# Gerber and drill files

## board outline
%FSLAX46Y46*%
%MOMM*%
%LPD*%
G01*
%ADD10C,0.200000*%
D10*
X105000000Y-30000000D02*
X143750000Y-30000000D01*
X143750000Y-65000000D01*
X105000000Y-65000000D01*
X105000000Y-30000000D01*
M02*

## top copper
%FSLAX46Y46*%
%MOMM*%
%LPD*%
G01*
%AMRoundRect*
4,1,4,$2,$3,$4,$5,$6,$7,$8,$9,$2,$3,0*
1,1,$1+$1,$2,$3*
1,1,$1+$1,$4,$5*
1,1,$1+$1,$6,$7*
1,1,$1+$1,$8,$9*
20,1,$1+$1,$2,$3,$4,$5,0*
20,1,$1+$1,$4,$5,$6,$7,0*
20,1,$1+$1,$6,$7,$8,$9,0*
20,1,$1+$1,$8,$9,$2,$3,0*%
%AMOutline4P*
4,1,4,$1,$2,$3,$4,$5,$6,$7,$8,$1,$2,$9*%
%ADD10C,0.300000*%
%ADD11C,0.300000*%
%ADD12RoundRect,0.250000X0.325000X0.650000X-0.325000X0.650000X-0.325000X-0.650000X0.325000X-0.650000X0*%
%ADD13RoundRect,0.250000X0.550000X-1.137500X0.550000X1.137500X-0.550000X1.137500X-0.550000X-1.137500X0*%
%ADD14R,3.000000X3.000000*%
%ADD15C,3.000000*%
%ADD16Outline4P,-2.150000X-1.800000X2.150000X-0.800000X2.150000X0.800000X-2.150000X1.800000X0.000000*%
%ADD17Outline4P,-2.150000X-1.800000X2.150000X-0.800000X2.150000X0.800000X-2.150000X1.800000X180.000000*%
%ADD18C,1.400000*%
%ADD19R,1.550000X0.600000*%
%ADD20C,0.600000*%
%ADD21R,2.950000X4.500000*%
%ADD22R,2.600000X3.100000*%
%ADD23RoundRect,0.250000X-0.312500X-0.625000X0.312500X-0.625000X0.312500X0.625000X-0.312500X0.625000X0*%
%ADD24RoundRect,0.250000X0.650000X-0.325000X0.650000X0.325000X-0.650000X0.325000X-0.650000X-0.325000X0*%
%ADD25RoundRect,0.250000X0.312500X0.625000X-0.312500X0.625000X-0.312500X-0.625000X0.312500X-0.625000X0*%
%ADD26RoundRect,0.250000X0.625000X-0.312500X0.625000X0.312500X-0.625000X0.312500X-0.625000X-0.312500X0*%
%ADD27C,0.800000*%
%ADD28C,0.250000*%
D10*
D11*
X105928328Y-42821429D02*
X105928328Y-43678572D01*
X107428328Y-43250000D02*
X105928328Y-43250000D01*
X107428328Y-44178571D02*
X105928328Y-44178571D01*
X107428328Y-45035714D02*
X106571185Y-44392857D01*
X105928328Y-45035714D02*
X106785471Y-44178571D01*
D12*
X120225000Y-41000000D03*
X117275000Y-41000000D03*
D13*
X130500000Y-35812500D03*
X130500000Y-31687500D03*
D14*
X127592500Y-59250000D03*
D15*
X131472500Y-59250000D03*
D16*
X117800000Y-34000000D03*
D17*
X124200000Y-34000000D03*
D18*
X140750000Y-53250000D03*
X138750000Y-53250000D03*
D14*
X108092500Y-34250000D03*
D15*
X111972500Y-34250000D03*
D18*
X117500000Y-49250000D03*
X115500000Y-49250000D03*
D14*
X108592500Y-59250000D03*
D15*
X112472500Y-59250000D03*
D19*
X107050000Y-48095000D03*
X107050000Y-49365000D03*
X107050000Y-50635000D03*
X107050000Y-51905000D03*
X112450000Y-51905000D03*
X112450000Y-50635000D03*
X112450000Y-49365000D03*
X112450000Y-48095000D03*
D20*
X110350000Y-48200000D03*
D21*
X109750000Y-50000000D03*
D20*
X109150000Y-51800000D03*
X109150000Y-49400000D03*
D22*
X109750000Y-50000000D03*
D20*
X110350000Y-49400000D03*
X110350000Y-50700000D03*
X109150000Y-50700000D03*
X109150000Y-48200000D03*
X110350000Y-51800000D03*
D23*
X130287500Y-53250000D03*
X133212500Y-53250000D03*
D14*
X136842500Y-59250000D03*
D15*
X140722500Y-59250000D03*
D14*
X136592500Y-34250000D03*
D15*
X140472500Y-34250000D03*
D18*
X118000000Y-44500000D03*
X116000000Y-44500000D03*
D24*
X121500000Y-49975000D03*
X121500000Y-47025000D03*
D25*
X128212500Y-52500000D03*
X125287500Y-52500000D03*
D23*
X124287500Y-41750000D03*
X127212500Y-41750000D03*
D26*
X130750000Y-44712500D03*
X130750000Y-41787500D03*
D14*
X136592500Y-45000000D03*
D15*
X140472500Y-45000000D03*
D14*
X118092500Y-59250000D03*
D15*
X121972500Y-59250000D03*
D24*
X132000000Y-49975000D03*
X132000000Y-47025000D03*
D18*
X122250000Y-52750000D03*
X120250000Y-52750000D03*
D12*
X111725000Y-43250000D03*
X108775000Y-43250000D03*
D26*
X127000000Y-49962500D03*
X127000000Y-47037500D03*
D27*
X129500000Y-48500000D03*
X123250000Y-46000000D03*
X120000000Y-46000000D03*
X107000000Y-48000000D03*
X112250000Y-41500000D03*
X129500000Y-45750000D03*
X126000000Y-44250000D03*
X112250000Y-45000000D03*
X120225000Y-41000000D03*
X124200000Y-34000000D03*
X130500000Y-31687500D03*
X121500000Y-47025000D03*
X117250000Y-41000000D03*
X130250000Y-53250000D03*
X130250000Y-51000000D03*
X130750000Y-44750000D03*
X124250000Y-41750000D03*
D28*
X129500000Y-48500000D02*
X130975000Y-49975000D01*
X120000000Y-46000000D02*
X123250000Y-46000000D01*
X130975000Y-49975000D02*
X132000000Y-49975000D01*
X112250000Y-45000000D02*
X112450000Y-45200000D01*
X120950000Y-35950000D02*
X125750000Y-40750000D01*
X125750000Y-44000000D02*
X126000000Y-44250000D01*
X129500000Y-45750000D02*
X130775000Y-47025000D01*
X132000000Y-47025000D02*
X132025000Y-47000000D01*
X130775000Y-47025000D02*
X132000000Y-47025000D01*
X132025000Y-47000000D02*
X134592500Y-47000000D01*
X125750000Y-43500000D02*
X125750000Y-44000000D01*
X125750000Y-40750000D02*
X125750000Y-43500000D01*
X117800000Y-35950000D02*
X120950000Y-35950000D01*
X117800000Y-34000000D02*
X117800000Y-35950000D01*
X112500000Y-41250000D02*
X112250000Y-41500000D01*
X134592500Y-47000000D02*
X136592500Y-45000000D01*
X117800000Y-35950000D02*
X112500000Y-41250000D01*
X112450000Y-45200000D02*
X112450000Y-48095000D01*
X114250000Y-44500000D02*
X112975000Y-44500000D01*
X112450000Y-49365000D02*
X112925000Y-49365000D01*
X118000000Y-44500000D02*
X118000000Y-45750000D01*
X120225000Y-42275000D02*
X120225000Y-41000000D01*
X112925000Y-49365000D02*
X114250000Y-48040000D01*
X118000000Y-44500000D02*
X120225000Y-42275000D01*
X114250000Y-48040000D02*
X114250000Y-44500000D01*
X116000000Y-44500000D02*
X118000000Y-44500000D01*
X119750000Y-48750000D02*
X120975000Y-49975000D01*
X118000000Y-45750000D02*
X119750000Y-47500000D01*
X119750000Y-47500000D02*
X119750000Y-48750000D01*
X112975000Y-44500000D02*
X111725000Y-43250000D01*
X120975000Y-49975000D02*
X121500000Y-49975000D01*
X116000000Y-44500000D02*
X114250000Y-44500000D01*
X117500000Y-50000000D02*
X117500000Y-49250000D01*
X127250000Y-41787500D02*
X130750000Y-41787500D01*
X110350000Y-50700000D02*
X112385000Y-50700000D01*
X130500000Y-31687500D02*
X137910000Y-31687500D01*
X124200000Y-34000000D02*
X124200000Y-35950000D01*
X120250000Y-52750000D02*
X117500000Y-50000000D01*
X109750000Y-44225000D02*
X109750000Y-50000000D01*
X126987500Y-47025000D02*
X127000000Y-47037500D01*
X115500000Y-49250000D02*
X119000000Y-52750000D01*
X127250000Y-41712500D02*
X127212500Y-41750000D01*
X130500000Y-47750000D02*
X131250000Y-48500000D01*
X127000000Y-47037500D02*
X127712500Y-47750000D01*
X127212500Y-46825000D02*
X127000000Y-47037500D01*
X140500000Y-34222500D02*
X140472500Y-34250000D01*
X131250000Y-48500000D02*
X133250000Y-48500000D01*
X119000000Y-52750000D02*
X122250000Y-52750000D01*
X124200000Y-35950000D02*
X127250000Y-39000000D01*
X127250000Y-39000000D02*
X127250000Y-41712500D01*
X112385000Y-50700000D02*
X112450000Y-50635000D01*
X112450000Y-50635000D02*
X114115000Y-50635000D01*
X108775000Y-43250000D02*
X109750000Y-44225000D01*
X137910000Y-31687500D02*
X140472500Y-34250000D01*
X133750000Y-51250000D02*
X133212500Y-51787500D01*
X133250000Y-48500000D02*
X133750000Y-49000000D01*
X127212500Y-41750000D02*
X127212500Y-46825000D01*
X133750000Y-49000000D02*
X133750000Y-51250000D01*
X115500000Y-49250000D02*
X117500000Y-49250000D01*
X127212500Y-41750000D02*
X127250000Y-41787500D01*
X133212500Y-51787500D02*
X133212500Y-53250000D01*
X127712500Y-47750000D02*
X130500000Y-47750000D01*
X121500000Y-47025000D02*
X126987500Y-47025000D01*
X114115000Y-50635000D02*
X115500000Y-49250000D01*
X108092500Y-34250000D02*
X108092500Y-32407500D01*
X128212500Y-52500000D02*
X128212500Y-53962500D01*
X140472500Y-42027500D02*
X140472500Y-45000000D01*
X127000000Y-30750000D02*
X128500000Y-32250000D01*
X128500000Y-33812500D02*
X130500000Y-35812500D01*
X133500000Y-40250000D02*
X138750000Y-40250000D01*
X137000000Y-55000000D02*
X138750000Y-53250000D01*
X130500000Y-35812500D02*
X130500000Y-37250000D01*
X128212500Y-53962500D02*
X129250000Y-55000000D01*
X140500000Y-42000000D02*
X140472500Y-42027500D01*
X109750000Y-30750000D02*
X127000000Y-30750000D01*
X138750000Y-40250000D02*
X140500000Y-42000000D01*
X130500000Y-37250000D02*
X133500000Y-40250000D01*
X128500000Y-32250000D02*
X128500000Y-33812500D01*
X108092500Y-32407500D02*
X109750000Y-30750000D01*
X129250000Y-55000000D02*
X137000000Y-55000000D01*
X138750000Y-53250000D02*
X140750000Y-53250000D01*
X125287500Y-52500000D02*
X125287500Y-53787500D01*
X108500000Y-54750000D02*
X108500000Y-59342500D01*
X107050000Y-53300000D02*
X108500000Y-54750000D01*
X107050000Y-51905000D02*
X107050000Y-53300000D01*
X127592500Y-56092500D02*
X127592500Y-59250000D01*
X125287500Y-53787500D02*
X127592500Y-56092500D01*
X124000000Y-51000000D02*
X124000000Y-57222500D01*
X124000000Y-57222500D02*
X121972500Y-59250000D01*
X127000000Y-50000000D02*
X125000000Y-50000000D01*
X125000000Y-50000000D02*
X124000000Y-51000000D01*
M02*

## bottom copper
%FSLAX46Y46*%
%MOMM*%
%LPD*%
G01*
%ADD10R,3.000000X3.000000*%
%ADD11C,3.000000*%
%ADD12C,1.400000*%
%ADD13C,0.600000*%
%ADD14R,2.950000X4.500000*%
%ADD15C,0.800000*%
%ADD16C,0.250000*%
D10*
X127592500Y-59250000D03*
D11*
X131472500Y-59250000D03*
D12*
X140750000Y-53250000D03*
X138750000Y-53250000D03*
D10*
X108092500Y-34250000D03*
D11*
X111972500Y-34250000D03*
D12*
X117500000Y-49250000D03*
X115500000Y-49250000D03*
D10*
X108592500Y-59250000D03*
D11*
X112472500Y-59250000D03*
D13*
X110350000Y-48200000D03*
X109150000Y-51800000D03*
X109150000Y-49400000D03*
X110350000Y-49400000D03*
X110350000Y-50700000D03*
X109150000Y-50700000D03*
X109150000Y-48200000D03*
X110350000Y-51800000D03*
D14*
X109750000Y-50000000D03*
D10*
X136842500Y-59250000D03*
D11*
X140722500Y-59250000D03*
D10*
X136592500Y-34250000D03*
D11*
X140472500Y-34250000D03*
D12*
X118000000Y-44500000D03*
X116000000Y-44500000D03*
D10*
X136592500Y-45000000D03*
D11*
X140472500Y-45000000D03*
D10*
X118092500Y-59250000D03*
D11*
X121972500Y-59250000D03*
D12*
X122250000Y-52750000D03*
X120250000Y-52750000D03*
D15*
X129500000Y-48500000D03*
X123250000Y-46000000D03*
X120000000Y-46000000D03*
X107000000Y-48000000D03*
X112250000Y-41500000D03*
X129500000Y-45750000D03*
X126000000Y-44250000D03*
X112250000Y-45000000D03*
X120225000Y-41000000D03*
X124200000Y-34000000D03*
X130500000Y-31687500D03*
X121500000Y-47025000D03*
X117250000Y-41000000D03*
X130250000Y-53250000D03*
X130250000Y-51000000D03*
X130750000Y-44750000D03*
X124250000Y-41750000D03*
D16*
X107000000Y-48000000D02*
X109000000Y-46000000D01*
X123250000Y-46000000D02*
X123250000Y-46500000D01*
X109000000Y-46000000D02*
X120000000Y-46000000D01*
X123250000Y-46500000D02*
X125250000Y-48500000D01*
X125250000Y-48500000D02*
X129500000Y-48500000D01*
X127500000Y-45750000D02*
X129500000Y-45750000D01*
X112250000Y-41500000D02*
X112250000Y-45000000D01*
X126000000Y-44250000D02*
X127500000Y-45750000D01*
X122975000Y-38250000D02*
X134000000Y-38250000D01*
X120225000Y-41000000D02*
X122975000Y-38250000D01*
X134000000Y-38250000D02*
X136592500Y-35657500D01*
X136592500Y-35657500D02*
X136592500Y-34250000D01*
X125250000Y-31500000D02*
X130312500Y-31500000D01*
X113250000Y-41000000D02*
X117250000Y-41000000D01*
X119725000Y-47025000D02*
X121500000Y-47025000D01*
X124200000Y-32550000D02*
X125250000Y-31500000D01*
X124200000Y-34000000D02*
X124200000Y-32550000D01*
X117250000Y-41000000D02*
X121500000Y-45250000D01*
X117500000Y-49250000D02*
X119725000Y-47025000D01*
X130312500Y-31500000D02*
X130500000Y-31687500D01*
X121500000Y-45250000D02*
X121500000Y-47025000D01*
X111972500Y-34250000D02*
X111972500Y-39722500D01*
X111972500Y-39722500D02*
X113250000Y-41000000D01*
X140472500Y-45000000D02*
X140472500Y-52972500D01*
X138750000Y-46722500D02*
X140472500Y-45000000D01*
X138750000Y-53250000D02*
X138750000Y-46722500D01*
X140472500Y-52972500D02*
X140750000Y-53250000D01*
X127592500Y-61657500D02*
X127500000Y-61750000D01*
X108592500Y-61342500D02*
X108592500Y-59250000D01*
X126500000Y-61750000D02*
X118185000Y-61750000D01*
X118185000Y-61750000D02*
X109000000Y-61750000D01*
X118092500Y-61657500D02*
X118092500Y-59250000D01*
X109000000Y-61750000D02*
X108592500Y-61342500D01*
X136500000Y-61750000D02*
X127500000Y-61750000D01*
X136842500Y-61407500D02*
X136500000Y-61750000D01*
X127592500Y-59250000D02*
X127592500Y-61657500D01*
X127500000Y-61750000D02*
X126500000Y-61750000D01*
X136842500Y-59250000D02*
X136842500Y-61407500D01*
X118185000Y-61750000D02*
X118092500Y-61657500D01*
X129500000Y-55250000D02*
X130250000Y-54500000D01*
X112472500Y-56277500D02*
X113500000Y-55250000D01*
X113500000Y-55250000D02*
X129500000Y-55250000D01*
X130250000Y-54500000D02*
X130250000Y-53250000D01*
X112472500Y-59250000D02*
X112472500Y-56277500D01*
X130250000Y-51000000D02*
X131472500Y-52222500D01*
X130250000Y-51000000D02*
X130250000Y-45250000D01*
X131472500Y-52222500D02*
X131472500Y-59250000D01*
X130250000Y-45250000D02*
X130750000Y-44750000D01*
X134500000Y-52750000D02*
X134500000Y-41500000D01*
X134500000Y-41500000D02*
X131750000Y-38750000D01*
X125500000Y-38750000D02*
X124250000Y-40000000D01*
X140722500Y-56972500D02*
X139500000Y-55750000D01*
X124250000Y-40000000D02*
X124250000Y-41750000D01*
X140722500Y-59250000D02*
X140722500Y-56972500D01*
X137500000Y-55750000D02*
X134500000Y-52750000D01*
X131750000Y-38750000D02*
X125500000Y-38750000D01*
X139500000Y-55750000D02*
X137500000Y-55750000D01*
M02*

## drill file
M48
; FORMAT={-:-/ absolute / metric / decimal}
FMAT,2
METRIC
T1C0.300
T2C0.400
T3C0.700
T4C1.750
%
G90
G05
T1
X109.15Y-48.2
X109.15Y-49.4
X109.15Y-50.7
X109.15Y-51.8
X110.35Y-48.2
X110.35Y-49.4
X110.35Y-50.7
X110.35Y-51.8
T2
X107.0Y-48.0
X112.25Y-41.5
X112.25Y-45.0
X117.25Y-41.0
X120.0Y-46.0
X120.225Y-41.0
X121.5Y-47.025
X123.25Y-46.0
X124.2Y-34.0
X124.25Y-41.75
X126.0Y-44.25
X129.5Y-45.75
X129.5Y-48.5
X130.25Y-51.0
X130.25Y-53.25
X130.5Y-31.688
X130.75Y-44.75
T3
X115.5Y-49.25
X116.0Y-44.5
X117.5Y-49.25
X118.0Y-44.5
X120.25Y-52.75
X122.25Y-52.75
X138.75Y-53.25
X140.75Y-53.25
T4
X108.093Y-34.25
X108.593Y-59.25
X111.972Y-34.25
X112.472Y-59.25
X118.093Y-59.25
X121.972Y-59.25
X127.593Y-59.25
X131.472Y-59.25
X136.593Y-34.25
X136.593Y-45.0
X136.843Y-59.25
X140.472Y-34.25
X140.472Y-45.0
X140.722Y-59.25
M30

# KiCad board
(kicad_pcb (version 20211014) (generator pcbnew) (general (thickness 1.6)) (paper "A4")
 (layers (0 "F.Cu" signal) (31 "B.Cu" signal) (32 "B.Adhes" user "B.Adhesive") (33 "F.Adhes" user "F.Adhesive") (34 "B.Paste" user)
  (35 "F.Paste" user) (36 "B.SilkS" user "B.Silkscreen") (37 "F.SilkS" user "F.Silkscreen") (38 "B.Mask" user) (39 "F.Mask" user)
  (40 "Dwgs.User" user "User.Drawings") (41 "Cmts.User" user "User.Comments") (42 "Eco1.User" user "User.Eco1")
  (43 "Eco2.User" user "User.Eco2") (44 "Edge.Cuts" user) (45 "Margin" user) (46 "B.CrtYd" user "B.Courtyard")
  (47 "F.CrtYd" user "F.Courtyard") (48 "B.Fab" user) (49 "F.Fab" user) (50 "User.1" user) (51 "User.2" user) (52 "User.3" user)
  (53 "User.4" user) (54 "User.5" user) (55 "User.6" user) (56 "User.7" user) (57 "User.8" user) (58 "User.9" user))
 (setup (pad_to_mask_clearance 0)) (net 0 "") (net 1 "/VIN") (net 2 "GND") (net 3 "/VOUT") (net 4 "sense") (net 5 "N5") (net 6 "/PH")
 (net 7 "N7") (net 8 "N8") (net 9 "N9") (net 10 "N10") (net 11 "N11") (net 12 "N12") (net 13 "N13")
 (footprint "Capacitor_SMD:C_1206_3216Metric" (layer "F.Cu") (at 118.75 41 180)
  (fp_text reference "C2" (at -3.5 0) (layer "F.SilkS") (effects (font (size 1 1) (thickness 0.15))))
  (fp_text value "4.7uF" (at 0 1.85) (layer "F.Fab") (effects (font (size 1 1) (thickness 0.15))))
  (pad "1" smd roundrect (at -1.475 0 180) (size 1.15 1.8) (layers "F.Cu" "F.Paste" "F.Mask") (roundrect_rratio 0.217391) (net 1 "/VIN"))
  (pad "2" smd roundrect (at 1.475 0 180) (size 1.15 1.8) (layers "F.Cu" "F.Paste" "F.Mask") (roundrect_rratio 0.217391) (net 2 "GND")))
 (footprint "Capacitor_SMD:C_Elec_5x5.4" (layer "F.Cu") (at 130.5 33.75 90)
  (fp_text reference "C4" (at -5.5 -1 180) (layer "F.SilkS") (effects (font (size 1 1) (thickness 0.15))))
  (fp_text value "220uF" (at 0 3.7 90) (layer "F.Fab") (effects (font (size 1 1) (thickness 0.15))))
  (pad "1" smd roundrect (at -2.0625 0 90) (size 2.775 1.6) (layers "F.Cu" "F.Paste" "F.Mask") (roundrect_rratio 0.15625) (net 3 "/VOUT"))
  (pad "2" smd roundrect (at 2.0625 0 90) (size 2.775 1.6) (layers "F.Cu" "F.Paste" "F.Mask") (roundrect_rratio 0.15625) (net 2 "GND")))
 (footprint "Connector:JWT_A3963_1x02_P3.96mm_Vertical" (layer "F.Cu") (at 127.5925 59.25)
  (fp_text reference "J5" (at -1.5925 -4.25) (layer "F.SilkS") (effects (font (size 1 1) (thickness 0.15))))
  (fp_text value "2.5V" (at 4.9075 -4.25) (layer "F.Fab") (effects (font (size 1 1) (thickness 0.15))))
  (pad "1" thru_hole rect (at 0 0) (size 3 3) (drill 1.75) (layers *.Cu *.Mask) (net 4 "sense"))
  (pad "2" thru_hole circle (at 3.88 0) (size 3 3) (drill 1.75) (layers *.Cu *.Mask) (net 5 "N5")))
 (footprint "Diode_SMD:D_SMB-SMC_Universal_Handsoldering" (layer "F.Cu") (at 121 34)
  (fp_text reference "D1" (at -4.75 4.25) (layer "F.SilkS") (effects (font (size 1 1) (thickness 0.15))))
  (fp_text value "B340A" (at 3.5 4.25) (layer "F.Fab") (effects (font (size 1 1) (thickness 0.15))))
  (pad "1" smd trapezoid (at -3.2 0) (size 4.3 2.6) (rect_delta 1 0) (layers "F.Cu" "F.Paste" "F.Mask") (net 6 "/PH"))
  (pad "2" smd trapezoid (at 3.2 0 180) (size 4.3 2.6) (rect_delta 1 0) (layers "F.Cu" "F.Paste" "F.Mask") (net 2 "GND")))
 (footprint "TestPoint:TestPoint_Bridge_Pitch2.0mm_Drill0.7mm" (layer "F.Cu") (at 138.75 53.25)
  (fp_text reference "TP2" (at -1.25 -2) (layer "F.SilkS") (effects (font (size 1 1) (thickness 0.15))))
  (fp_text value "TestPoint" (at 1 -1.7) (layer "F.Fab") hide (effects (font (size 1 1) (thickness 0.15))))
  (pad "1" thru_hole circle (at 2 0) (size 1.4 1.4) (drill 0.7) (layers *.Cu *.Mask) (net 3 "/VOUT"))
  (pad "1" thru_hole circle (at 0 0) (size 1.4 1.4) (drill 0.7) (layers *.Cu *.Mask) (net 3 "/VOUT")))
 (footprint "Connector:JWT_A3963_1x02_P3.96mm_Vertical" (layer "F.Cu") (at 108.0925 34.25)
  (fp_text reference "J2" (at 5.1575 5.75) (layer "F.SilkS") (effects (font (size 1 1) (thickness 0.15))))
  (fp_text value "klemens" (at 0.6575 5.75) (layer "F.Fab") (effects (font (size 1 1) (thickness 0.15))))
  (pad "1" thru_hole rect (at 0 0) (size 3 3) (drill 1.75) (layers *.Cu *.Mask) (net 3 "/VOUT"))
  (pad "2" thru_hole circle (at 3.88 0) (size 3 3) (drill 1.75) (layers *.Cu *.Mask) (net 2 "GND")))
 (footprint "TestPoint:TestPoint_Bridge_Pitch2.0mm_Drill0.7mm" (layer "F.Cu") (at 115.5 49.25)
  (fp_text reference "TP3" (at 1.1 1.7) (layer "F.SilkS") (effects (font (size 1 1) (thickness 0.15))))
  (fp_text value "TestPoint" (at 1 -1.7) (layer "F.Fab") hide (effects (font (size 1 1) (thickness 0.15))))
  (pad "1" thru_hole circle (at 2 0) (size 1.4 1.4) (drill 0.7) (layers *.Cu *.Mask) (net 2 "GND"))
  (pad "1" thru_hole circle (at 0 0) (size 1.4 1.4) (drill 0.7) (layers *.Cu *.Mask) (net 2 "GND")))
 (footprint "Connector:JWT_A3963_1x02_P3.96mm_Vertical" (layer "F.Cu") (at 108.5925 59.25)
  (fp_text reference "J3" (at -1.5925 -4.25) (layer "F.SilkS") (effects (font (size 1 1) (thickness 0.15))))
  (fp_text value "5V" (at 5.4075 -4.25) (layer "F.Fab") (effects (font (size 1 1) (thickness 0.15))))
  (pad "1" thru_hole rect (at 0 0) (size 3 3) (drill 1.75) (layers *.Cu *.Mask) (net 4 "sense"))
  (pad "2" thru_hole circle (at 3.88 0) (size 3 3) (drill 1.75) (layers *.Cu *.Mask) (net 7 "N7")))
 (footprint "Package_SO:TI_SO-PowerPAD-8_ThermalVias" (layer "F.Cu") (at 109.75 50)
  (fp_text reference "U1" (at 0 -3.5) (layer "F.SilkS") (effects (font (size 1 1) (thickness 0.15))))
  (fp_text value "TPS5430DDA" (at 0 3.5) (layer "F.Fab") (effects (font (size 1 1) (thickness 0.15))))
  (pad "1" smd rect (at -2.7 -1.905) (size 1.55 0.6) (layers "F.Cu" "F.Paste" "F.Mask") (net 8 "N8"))
  (pad "2" smd rect (at -2.7 -0.635) (size 1.55 0.6) (layers "F.Cu" "F.Paste" "F.Mask") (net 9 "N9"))
  (pad "3" smd rect (at -2.7 0.635) (size 1.55 0.6) (layers "F.Cu" "F.Paste" "F.Mask") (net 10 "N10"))
  (pad "4" smd rect (at -2.7 1.905) (size 1.55 0.6) (layers "F.Cu" "F.Paste" "F.Mask") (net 4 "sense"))
  (pad "5" smd rect (at 2.7 1.905) (size 1.55 0.6) (layers "F.Cu" "F.Paste" "F.Mask") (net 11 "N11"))
  (pad "6" smd rect (at 2.7 0.635) (size 1.55 0.6) (layers "F.Cu" "F.Paste" "F.Mask") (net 2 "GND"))
  (pad "7" smd rect (at 2.7 -0.635) (size 1.55 0.6) (layers "F.Cu" "F.Paste" "F.Mask") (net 1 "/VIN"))
  (pad "8" smd rect (at 2.7 -1.905) (size 1.55 0.6) (layers "F.Cu" "F.Paste" "F.Mask") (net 6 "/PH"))
  (pad "9" thru_hole circle (at 0.6 -1.8) (size 0.6 0.6) (drill 0.3) (layers *.Cu) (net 2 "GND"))
  (pad "9" smd rect (at 0 0) (size 2.95 4.5) (layers "F.Cu") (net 2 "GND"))
  (pad "9" thru_hole circle (at -0.6 1.8) (size 0.6 0.6) (drill 0.3) (layers *.Cu) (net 2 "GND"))
  (pad "9" thru_hole circle (at -0.6 -0.6) (size 0.6 0.6) (drill 0.3) (layers *.Cu) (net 2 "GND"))
  (pad "9" smd rect (at 0 0) (size 2.6 3.1) (layers "F.Cu" "F.Paste" "F.Mask") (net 2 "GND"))
  (pad "9" thru_hole circle (at 0.6 -0.6) (size 0.6 0.6) (drill 0.3) (layers *.Cu) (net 2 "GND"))
  (pad "9" thru_hole circle (at 0.6 0.7) (size 0.6 0.6) (drill 0.3) (layers *.Cu) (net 2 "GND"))
  (pad "9" thru_hole circle (at -0.6 0.7) (size 0.6 0.6) (drill 0.3) (layers *.Cu) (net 2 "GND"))
  (pad "9" thru_hole circle (at -0.6 -1.8) (size 0.6 0.6) (drill 0.3) (layers *.Cu) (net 2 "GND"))
  (pad "9" thru_hole circle (at 0.6 1.8) (size 0.6 0.6) (drill 0.3) (layers *.Cu) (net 2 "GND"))
  (pad "9" smd rect (at 0 0) (size 2.95 4.5) (layers "B.Cu") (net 2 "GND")))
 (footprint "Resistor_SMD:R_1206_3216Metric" (layer "F.Cu") (at 131.75 53.25)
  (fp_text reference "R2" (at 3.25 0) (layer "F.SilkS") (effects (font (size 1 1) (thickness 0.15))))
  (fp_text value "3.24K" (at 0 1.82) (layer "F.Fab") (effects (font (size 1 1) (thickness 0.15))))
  (pad "1" smd roundrect (at -1.4625 0) (size 1.125 1.75) (layers "F.Cu" "F.Paste" "F.Mask") (roundrect_rratio 0.222222) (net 7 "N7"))
  (pad "2" smd roundrect (at 1.4625 0) (size 1.125 1.75) (layers "F.Cu" "F.Paste" "F.Mask") (roundrect_rratio 0.222222) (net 2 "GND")))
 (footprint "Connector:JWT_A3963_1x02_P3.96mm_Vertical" (layer "F.Cu") (at 136.8425 59.25)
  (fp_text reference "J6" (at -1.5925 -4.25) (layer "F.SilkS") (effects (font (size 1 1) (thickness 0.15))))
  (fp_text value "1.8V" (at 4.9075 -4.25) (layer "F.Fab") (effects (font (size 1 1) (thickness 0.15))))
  (pad "1" thru_hole rect (at 0 0) (size 3 3) (drill 1.75) (layers *.Cu *.Mask) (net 4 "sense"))
  (pad "2" thru_hole circle (at 3.88 0) (size 3 3) (drill 1.75) (layers *.Cu *.Mask) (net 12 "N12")))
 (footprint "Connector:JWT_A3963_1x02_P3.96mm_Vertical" (layer "F.Cu") (at 136.5925 34.25)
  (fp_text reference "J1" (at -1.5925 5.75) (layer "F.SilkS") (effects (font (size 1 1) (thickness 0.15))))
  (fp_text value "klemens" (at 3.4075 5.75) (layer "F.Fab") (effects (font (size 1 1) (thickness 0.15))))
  (pad "1" thru_hole rect (at 0 0) (size 3 3) (drill 1.75) (layers *.Cu *.Mask) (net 1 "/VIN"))
  (pad "2" thru_hole circle (at 3.88 0) (size 3 3) (drill 1.75) (layers *.Cu *.Mask) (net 2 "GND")))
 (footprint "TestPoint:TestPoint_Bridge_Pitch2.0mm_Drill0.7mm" (layer "F.Cu") (at 116 44.5)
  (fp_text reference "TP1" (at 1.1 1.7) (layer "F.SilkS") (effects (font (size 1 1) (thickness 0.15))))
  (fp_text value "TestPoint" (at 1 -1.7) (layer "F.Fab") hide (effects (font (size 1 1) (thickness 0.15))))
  (pad "1" thru_hole circle (at 2 0) (size 1.4 1.4) (drill 0.7) (layers *.Cu *.Mask) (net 1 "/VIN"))
  (pad "1" thru_hole circle (at 0 0) (size 1.4 1.4) (drill 0.7) (layers *.Cu *.Mask) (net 1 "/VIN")))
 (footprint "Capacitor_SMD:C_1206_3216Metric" (layer "F.Cu") (at 121.5 48.5 90)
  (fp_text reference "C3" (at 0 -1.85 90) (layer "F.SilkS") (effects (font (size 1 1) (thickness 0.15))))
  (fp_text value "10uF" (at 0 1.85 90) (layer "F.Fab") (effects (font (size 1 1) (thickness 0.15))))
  (pad "1" smd roundrect (at -1.475 0 90) (size 1.15 1.8) (layers "F.Cu" "F.Paste" "F.Mask") (roundrect_rratio 0.217391) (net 1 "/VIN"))
  (pad "2" smd roundrect (at 1.475 0 90) (size 1.15 1.8) (layers "F.Cu" "F.Paste" "F.Mask") (roundrect_rratio 0.217391) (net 2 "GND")))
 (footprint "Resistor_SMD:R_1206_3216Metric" (layer "F.Cu") (at 126.75 52.5 180)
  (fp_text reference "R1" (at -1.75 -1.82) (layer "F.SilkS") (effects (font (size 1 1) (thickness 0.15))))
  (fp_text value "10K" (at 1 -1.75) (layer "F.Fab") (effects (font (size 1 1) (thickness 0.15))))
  (pad "1" smd roundrect (at -1.4625 0 180) (size 1.125 1.75) (layers "F.Cu" "F.Paste" "F.Mask") (roundrect_rratio 0.222222) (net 3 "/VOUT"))
  (pad "2" smd roundrect (at 1.4625 0 180) (size 1.125 1.75) (layers "F.Cu" "F.Paste" "F.Mask") (roundrect_rratio 0.222222) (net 4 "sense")))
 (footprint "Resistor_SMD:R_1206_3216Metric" (layer "F.Cu") (at 125.75 41.75)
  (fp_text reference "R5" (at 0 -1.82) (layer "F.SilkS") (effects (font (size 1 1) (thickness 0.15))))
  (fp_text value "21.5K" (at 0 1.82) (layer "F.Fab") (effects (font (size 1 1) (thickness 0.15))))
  (pad "1" smd roundrect (at -1.4625 0) (size 1.125 1.75) (layers "F.Cu" "F.Paste" "F.Mask") (roundrect_rratio 0.222222) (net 12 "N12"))
  (pad "2" smd roundrect (at 1.4625 0) (size 1.125 1.75) (layers "F.Cu" "F.Paste" "F.Mask") (roundrect_rratio 0.222222) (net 2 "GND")))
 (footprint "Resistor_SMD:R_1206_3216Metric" (layer "F.Cu") (at 130.75 43.25 90)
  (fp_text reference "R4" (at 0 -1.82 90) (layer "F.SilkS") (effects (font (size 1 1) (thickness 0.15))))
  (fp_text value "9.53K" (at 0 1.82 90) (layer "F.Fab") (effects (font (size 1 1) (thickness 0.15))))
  (pad "1" smd roundrect (at -1.4625 0 90) (size 1.125 1.75) (layers "F.Cu" "F.Paste" "F.Mask") (roundrect_rratio 0.222222) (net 5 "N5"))
  (pad "2" smd roundrect (at 1.4625 0 90) (size 1.125 1.75) (layers "F.Cu" "F.Paste" "F.Mask") (roundrect_rratio 0.222222) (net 2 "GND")))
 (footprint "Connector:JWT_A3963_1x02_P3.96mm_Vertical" (layer "F.Cu") (at 136.5925 45)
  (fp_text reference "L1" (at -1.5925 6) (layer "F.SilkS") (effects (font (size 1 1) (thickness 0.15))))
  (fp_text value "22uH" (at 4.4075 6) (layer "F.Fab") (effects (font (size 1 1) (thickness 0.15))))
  (pad "1" thru_hole rect (at 0 0) (size 3 3) (drill 1.75) (layers *.Cu *.Mask) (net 6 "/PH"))
  (pad "2" thru_hole circle (at 3.88 0) (size 3 3) (drill 1.75) (layers *.Cu *.Mask) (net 3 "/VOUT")))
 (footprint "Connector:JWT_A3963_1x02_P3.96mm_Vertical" (layer "F.Cu") (at 118.0925 59.25)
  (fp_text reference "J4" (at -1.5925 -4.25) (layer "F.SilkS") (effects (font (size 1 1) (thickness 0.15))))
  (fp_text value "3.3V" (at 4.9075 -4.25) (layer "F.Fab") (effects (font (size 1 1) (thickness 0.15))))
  (pad "1" thru_hole rect (at 0 0) (size 3 3) (drill 1.75) (layers *.Cu *.Mask) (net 4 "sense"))
  (pad "2" thru_hole circle (at 3.88 0) (size 3 3) (drill 1.75) (layers *.Cu *.Mask) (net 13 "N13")))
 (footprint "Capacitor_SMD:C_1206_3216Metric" (layer "F.Cu") (at 132 48.5 90)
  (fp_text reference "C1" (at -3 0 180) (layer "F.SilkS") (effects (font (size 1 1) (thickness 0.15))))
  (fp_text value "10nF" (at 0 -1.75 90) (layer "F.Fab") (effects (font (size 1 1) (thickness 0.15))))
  (pad "1" smd roundrect (at -1.475 0 90) (size 1.15 1.8) (layers "F.Cu" "F.Paste" "F.Mask") (roundrect_rratio 0.217391) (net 8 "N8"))
  (pad "2" smd roundrect (at 1.475 0 90) (size 1.15 1.8) (layers "F.Cu" "F.Paste" "F.Mask") (roundrect_rratio 0.217391) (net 6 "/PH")))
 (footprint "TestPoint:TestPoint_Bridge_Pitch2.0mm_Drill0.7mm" (layer "F.Cu") (at 120.25 52.75)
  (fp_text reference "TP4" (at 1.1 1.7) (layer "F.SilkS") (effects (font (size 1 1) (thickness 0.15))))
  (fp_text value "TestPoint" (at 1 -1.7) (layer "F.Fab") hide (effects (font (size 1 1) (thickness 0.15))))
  (pad "1" thru_hole circle (at 2 0) (size 1.4 1.4) (drill 0.7) (layers *.Cu *.Mask) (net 2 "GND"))
  (pad "1" thru_hole circle (at 0 0) (size 1.4 1.4) (drill 0.7) (layers *.Cu *.Mask) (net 2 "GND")))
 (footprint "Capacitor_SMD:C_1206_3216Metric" (layer "F.Cu") (at 110.25 43.25 180)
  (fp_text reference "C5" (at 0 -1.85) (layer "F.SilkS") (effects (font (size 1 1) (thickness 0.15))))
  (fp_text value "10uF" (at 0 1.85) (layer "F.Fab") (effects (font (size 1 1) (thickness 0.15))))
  (pad "1" smd roundrect (at -1.475 0 180) (size 1.15 1.8) (layers "F.Cu" "F.Paste" "F.Mask") (roundrect_rratio 0.217391) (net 1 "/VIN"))
  (pad "2" smd roundrect (at 1.475 0 180) (size 1.15 1.8) (layers "F.Cu" "F.Paste" "F.Mask") (roundrect_rratio 0.217391) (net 2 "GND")))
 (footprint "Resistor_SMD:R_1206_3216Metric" (layer "F.Cu") (at 127 48.5 90)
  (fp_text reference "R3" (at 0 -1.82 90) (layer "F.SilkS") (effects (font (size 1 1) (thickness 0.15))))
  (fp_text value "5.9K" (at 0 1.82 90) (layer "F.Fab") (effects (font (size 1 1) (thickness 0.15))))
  (pad "1" smd roundrect (at -1.4625 0 90) (size 1.125 1.75) (layers "F.Cu" "F.Paste" "F.Mask") (roundrect_rratio 0.222222) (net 13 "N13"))
  (pad "2" smd roundrect (at 1.4625 0 90) (size 1.125 1.75) (layers "F.Cu" "F.Paste" "F.Mask") (roundrect_rratio 0.222222) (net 2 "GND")))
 (gr_rect (start 105 65) (end 143.75 30) (layer "Edge.Cuts") (width 0.2) (fill none))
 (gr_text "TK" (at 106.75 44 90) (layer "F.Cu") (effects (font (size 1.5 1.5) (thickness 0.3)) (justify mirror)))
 (segment (start 129.5 48.5) (end 130.975 49.975) (width 0.25) (layer "F.Cu") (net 8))
 (segment (start 120 46) (end 123.25 46) (width 0.25) (layer "F.Cu") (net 8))
 (segment (start 130.975 49.975) (end 132 49.975) (width 0.25) (layer "F.Cu") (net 8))
 (via (at 129.5 48.5) (size 0.8) (drill 0.4) (layers "F.Cu" "B.Cu") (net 8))
 (via (at 123.25 46) (size 0.8) (drill 0.4) (layers "F.Cu" "B.Cu") (free) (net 8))
 (via (at 120 46) (size 0.8) (drill 0.4) (layers "F.Cu" "B.Cu") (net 8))
 (via (at 107 48) (size 0.8) (drill 0.4) (layers "F.Cu" "B.Cu") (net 8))
 (segment (start 107 48) (end 109 46) (width 0.25) (layer "B.Cu") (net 8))
 (segment (start 123.25 46) (end 123.25 46.5) (width 0.25) (layer "B.Cu") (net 8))
 (segment (start 109 46) (end 120 46) (width 0.25) (layer "B.Cu") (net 8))
 (segment (start 123.25 46.5) (end 125.25 48.5) (width 0.25) (layer "B.Cu") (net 8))
 (segment (start 125.25 48.5) (end 129.5 48.5) (width 0.25) (layer "B.Cu") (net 8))
 (segment (start 112.25 45) (end 112.45 45.2) (width 0.25) (layer "F.Cu") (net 6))
 (segment (start 120.95 35.95) (end 125.75 40.75) (width 0.25) (layer "F.Cu") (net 6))
 (segment (start 125.75 44) (end 126 44.25) (width 0.25) (layer "F.Cu") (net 6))
 (segment (start 129.5 45.75) (end 130.775 47.025) (width 0.25) (layer "F.Cu") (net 6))
 (segment (start 132 47.025) (end 132.025 47) (width 0.25) (layer "F.Cu") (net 6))
 (segment (start 130.775 47.025) (end 132 47.025) (width 0.25) (layer "F.Cu") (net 6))
 (segment (start 132.025 47) (end 134.5925 47) (width 0.25) (layer "F.Cu") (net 6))
 (segment (start 125.75 43.5) (end 125.75 44) (width 0.25) (layer "F.Cu") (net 6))
 (segment (start 125.75 40.75) (end 125.75 43.5) (width 0.25) (layer "F.Cu") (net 6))
 (segment (start 117.8 35.95) (end 120.95 35.95) (width 0.25) (layer "F.Cu") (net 6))
 (segment (start 117.8 34) (end 117.8 35.95) (width 0.25) (layer "F.Cu") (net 6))
 (segment (start 112.5 41.25) (end 112.25 41.5) (width 0.25) (layer "F.Cu") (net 6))
 (segment (start 134.5925 47) (end 136.5925 45) (width 0.25) (layer "F.Cu") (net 6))
 (segment (start 117.8 35.95) (end 112.5 41.25) (width 0.25) (layer "F.Cu") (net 6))
 (segment (start 112.45 45.2) (end 112.45 48.095) (width 0.25) (layer "F.Cu") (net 6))
 (via (at 112.25 41.5) (size 0.8) (drill 0.4) (layers "F.Cu" "B.Cu") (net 6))
 (via (at 129.5 45.75) (size 0.8) (drill 0.4) (layers "F.Cu" "B.Cu") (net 6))
 (via (at 126 44.25) (size 0.8) (drill 0.4) (layers "F.Cu" "B.Cu") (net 6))
 (via (at 112.25 45) (size 0.8) (drill 0.4) (layers "F.Cu" "B.Cu") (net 6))
 (segment (start 127.5 45.75) (end 129.5 45.75) (width 0.25) (layer "B.Cu") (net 6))
 (segment (start 112.25 41.5) (end 112.25 45) (width 0.25) (layer "B.Cu") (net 6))
 (segment (start 126 44.25) (end 127.5 45.75) (width 0.25) (layer "B.Cu") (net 6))
 (segment (start 114.25 44.5) (end 112.975 44.5) (width 0.25) (layer "F.Cu") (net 1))
 (segment (start 112.45 49.365) (end 112.925 49.365) (width 0.25) (layer "F.Cu") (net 1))
 (segment (start 118 44.5) (end 118 45.75) (width 0.25) (layer "F.Cu") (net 1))
 (segment (start 120.225 42.275) (end 120.225 41) (width 0.25) (layer "F.Cu") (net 1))
 (segment (start 112.925 49.365) (end 114.25 48.04) (width 0.25) (layer "F.Cu") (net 1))
 (segment (start 118 44.5) (end 120.225 42.275) (width 0.25) (layer "F.Cu") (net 1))
 (segment (start 114.25 48.04) (end 114.25 44.5) (width 0.25) (layer "F.Cu") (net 1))
 (segment (start 116 44.5) (end 118 44.5) (width 0.25) (layer "F.Cu") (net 1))
 (segment (start 119.75 48.75) (end 120.975 49.975) (width 0.25) (layer "F.Cu") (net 1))
 (segment (start 118 45.75) (end 119.75 47.5) (width 0.25) (layer "F.Cu") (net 1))
 (segment (start 119.75 47.5) (end 119.75 48.75) (width 0.25) (layer "F.Cu") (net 1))
 (segment (start 112.975 44.5) (end 111.725 43.25) (width 0.25) (layer "F.Cu") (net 1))
 (segment (start 120.975 49.975) (end 121.5 49.975) (width 0.25) (layer "F.Cu") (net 1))
 (segment (start 116 44.5) (end 114.25 44.5) (width 0.25) (layer "F.Cu") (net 1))
 (via (at 120.225 41) (size 0.8) (drill 0.4) (layers "F.Cu" "B.Cu") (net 1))
 (segment (start 122.975 38.25) (end 134 38.25) (width 0.25) (layer "B.Cu") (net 1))
 (segment (start 120.225 41) (end 122.975 38.25) (width 0.25) (layer "B.Cu") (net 1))
 (segment (start 134 38.25) (end 136.5925 35.6575) (width 0.25) (layer "B.Cu") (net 1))
 (segment (start 136.5925 35.6575) (end 136.5925 34.25) (width 0.25) (layer "B.Cu") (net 1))
 (segment (start 117.5 50) (end 117.5 49.25) (width 0.25) (layer "F.Cu") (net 2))
 (segment (start 127.25 41.7875) (end 130.75 41.7875) (width 0.25) (layer "F.Cu") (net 2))
 (segment (start 110.35 50.7) (end 112.385 50.7) (width 0.25) (layer "F.Cu") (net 2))
 (segment (start 130.5 31.6875) (end 137.91 31.6875) (width 0.25) (layer "F.Cu") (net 2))
 (segment (start 124.2 34) (end 124.2 35.95) (width 0.25) (layer "F.Cu") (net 2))
 (segment (start 120.25 52.75) (end 117.5 50) (width 0.25) (layer "F.Cu") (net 2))
 (segment (start 109.75 44.225) (end 109.75 50) (width 0.25) (layer "F.Cu") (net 2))
 (segment (start 126.9875 47.025) (end 127 47.0375) (width 0.25) (layer "F.Cu") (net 2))
 (segment (start 115.5 49.25) (end 119 52.75) (width 0.25) (layer "F.Cu") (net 2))
 (segment (start 127.25 41.7125) (end 127.2125 41.75) (width 0.25) (layer "F.Cu") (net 2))
 (segment (start 130.5 47.75) (end 131.25 48.5) (width 0.25) (layer "F.Cu") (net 2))
 (segment (start 127 47.0375) (end 127.7125 47.75) (width 0.25) (layer "F.Cu") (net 2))
 (segment (start 127.2125 46.825) (end 127 47.0375) (width 0.25) (layer "F.Cu") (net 2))
 (segment (start 140.5 34.2225) (end 140.4725 34.25) (width 0.25) (layer "F.Cu") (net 2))
 (segment (start 131.25 48.5) (end 133.25 48.5) (width 0.25) (layer "F.Cu") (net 2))
 (segment (start 119 52.75) (end 122.25 52.75) (width 0.25) (layer "F.Cu") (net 2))
 (segment (start 124.2 35.95) (end 127.25 39) (width 0.25) (layer "F.Cu") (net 2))
 (segment (start 127.25 39) (end 127.25 41.7125) (width 0.25) (layer "F.Cu") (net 2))
 (segment (start 112.385 50.7) (end 112.45 50.635) (width 0.25) (layer "F.Cu") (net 2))
 (segment (start 112.45 50.635) (end 114.115 50.635) (width 0.25) (layer "F.Cu") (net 2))
 (segment (start 108.775 43.25) (end 109.75 44.225) (width 0.25) (layer "F.Cu") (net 2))
 (segment (start 137.91 31.6875) (end 140.4725 34.25) (width 0.25) (layer "F.Cu") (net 2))
 (segment (start 133.75 51.25) (end 133.2125 51.7875) (width 0.25) (layer "F.Cu") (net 2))
 (segment (start 133.25 48.5) (end 133.75 49) (width 0.25) (layer "F.Cu") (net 2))
 (segment (start 127.2125 41.75) (end 127.2125 46.825) (width 0.25) (layer "F.Cu") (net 2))
 (segment (start 133.75 49) (end 133.75 51.25) (width 0.25) (layer "F.Cu") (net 2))
 (segment (start 115.5 49.25) (end 117.5 49.25) (width 0.25) (layer "F.Cu") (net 2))
 (segment (start 127.2125 41.75) (end 127.25 41.7875) (width 0.25) (layer "F.Cu") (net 2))
 (segment (start 133.2125 51.7875) (end 133.2125 53.25) (width 0.25) (layer "F.Cu") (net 2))
 (segment (start 127.7125 47.75) (end 130.5 47.75) (width 0.25) (layer "F.Cu") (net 2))
 (segment (start 121.5 47.025) (end 126.9875 47.025) (width 0.25) (layer "F.Cu") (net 2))
 (segment (start 114.115 50.635) (end 115.5 49.25) (width 0.25) (layer "F.Cu") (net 2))
 (via (at 124.2 34) (size 0.8) (drill 0.4) (layers "F.Cu" "B.Cu") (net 2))
 (via (at 130.5 31.6875) (size 0.8) (drill 0.4) (layers "F.Cu" "B.Cu") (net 2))
 (via (at 121.5 47.025) (size 0.8) (drill 0.4) (layers "F.Cu" "B.Cu") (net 2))
 (via (at 117.25 41) (size 0.8) (drill 0.4) (layers "F.Cu" "B.Cu") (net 2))
 (segment (start 125.25 31.5) (end 130.3125 31.5) (width 0.25) (layer "B.Cu") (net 2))
 (segment (start 113.25 41) (end 117.25 41) (width 0.25) (layer "B.Cu") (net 2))
 (segment (start 119.725 47.025) (end 121.5 47.025) (width 0.25) (layer "B.Cu") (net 2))
 (segment (start 124.2 32.55) (end 125.25 31.5) (width 0.25) (layer "B.Cu") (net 2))
 (segment (start 124.2 34) (end 124.2 32.55) (width 0.25) (layer "B.Cu") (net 2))
 (segment (start 117.25 41) (end 121.5 45.25) (width 0.25) (layer "B.Cu") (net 2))
 (segment (start 117.5 49.25) (end 119.725 47.025) (width 0.25) (layer "B.Cu") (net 2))
 (segment (start 130.3125 31.5) (end 130.5 31.6875) (width 0.25) (layer "B.Cu") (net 2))
 (segment (start 121.5 45.25) (end 121.5 47.025) (width 0.25) (layer "B.Cu") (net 2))
 (segment (start 111.9725 34.25) (end 111.9725 39.7225) (width 0.25) (layer "B.Cu") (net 2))
 (segment (start 111.9725 39.7225) (end 113.25 41) (width 0.25) (layer "B.Cu") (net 2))
 (segment (start 108.0925 34.25) (end 108.0925 32.4075) (width 0.25) (layer "F.Cu") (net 3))
 (segment (start 128.2125 52.5) (end 128.2125 53.9625) (width 0.25) (layer "F.Cu") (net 3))
 (segment (start 140.4725 42.0275) (end 140.4725 45) (width 0.25) (layer "F.Cu") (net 3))
 (segment (start 127 30.75) (end 128.5 32.25) (width 0.25) (layer "F.Cu") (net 3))
 (segment (start 128.5 33.8125) (end 130.5 35.8125) (width 0.25) (layer "F.Cu") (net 3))
 (segment (start 133.5 40.25) (end 138.75 40.25) (width 0.25) (layer "F.Cu") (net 3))
 (segment (start 137 55) (end 138.75 53.25) (width 0.25) (layer "F.Cu") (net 3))
 (segment (start 130.5 35.8125) (end 130.5 37.25) (width 0.25) (layer "F.Cu") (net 3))
 (segment (start 128.2125 53.9625) (end 129.25 55) (width 0.25) (layer "F.Cu") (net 3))
 (segment (start 140.5 42) (end 140.4725 42.0275) (width 0.25) (layer "F.Cu") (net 3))
 (segment (start 109.75 30.75) (end 127 30.75) (width 0.25) (layer "F.Cu") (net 3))
 (segment (start 138.75 40.25) (end 140.5 42) (width 0.25) (layer "F.Cu") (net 3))
 (segment (start 130.5 37.25) (end 133.5 40.25) (width 0.25) (layer "F.Cu") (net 3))
 (segment (start 128.5 32.25) (end 128.5 33.8125) (width 0.25) (layer "F.Cu") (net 3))
 (segment (start 108.0925 32.4075) (end 109.75 30.75) (width 0.25) (layer "F.Cu") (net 3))
 (segment (start 129.25 55) (end 137 55) (width 0.25) (layer "F.Cu") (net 3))
 (segment (start 138.75 53.25) (end 140.75 53.25) (width 0.25) (layer "F.Cu") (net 3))
 (segment (start 140.4725 45) (end 140.4725 52.9725) (width 0.25) (layer "B.Cu") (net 3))
 (segment (start 138.75 46.7225) (end 140.4725 45) (width 0.25) (layer "B.Cu") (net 3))
 (segment (start 138.75 53.25) (end 138.75 46.7225) (width 0.25) (layer "B.Cu") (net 3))
 (segment (start 140.4725 52.9725) (end 140.75 53.25) (width 0.25) (layer "B.Cu") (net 3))
 (segment (start 125.2875 52.5) (end 125.2875 53.7875) (width 0.25) (layer "F.Cu") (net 4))
 (segment (start 108.5 54.75) (end 108.5 59.3425) (width 0.25) (layer "F.Cu") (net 4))
 (segment (start 107.05 53.3) (end 108.5 54.75) (width 0.25) (layer "F.Cu") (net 4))
 (segment (start 107.05 51.905) (end 107.05 53.3) (width 0.25) (layer "F.Cu") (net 4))
 (segment (start 127.5925 56.0925) (end 127.5925 59.25) (width 0.25) (layer "F.Cu") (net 4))
 (segment (start 125.2875 53.7875) (end 127.5925 56.0925) (width 0.25) (layer "F.Cu") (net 4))
 (segment (start 127.5925 61.6575) (end 127.5 61.75) (width 0.25) (layer "B.Cu") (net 4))
 (segment (start 108.5925 61.3425) (end 108.5925 59.25) (width 0.25) (layer "B.Cu") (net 4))
 (segment (start 126.5 61.75) (end 118.185 61.75) (width 0.25) (layer "B.Cu") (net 4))
 (segment (start 118.185 61.75) (end 109 61.75) (width 0.25) (layer "B.Cu") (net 4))
 (segment (start 118.0925 61.6575) (end 118.0925 59.25) (width 0.25) (layer "B.Cu") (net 4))
 (segment (start 109 61.75) (end 108.5925 61.3425) (width 0.25) (layer "B.Cu") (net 4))
 (segment (start 136.5 61.75) (end 127.5 61.75) (width 0.25) (layer "B.Cu") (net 4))
 (segment (start 136.8425 61.4075) (end 136.5 61.75) (width 0.25) (layer "B.Cu") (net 4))
 (segment (start 127.5925 59.25) (end 127.5925 61.6575) (width 0.25) (layer "B.Cu") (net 4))
 (segment (start 127.5 61.75) (end 126.5 61.75) (width 0.25) (layer "B.Cu") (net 4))
 (segment (start 136.8425 59.25) (end 136.8425 61.4075) (width 0.25) (layer "B.Cu") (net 4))
 (segment (start 118.185 61.75) (end 118.0925 61.6575) (width 0.25) (layer "B.Cu") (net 4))
 (via (at 130.25 53.25) (size 0.8) (drill 0.4) (layers "F.Cu" "B.Cu") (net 7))
 (segment (start 129.5 55.25) (end 130.25 54.5) (width 0.25) (layer "B.Cu") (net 7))
 (segment (start 112.4725 56.2775) (end 113.5 55.25) (width 0.25) (layer "B.Cu") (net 7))
 (segment (start 113.5 55.25) (end 129.5 55.25) (width 0.25) (layer "B.Cu") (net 7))
 (segment (start 130.25 54.5) (end 130.25 53.25) (width 0.25) (layer "B.Cu") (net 7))
 (segment (start 112.4725 59.25) (end 112.4725 56.2775) (width 0.25) (layer "B.Cu") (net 7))
 (segment (start 124 51) (end 124 57.2225) (width 0.25) (layer "F.Cu") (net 13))
 (segment (start 124 57.2225) (end 121.9725 59.25) (width 0.25) (layer "F.Cu") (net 13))
 (segment (start 127 50) (end 125 50) (width 0.25) (layer "F.Cu") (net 13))
 (segment (start 125 50) (end 124 51) (width 0.25) (layer "F.Cu") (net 13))
 (via (at 130.25 51) (size 0.8) (drill 0.4) (layers "F.Cu" "B.Cu") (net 5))
 (via (at 130.75 44.75) (size 0.8) (drill 0.4) (layers "F.Cu" "B.Cu") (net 5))
 (segment (start 130.25 51) (end 131.4725 52.2225) (width 0.25) (layer "B.Cu") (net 5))
 (segment (start 130.25 51) (end 130.25 45.25) (width 0.25) (layer "B.Cu") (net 5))
 (segment (start 131.4725 52.2225) (end 131.4725 59.25) (width 0.25) (layer "B.Cu") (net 5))
 (segment (start 130.25 45.25) (end 130.75 44.75) (width 0.25) (layer "B.Cu") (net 5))
 (via (at 124.25 41.75) (size 0.8) (drill 0.4) (layers "F.Cu" "B.Cu") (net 12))
 (segment (start 134.5 52.75) (end 134.5 41.5) (width 0.25) (layer "B.Cu") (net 12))
 (segment (start 134.5 41.5) (end 131.75 38.75) (width 0.25) (layer "B.Cu") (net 12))
 (segment (start 125.5 38.75) (end 124.25 40) (width 0.25) (layer "B.Cu") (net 12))
 (segment (start 140.7225 56.9725) (end 139.5 55.75) (width 0.25) (layer "B.Cu") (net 12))
 (segment (start 124.25 40) (end 124.25 41.75) (width 0.25) (layer "B.Cu") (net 12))
 (segment (start 140.7225 59.25) (end 140.7225 56.9725) (width 0.25) (layer "B.Cu") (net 12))
 (segment (start 137.5 55.75) (end 134.5 52.75) (width 0.25) (layer "B.Cu") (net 12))
 (segment (start 131.75 38.75) (end 125.5 38.75) (width 0.25) (layer "B.Cu") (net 12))
 (segment (start 139.5 55.75) (end 137.5 55.75) (width 0.25) (layer "B.Cu") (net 12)))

